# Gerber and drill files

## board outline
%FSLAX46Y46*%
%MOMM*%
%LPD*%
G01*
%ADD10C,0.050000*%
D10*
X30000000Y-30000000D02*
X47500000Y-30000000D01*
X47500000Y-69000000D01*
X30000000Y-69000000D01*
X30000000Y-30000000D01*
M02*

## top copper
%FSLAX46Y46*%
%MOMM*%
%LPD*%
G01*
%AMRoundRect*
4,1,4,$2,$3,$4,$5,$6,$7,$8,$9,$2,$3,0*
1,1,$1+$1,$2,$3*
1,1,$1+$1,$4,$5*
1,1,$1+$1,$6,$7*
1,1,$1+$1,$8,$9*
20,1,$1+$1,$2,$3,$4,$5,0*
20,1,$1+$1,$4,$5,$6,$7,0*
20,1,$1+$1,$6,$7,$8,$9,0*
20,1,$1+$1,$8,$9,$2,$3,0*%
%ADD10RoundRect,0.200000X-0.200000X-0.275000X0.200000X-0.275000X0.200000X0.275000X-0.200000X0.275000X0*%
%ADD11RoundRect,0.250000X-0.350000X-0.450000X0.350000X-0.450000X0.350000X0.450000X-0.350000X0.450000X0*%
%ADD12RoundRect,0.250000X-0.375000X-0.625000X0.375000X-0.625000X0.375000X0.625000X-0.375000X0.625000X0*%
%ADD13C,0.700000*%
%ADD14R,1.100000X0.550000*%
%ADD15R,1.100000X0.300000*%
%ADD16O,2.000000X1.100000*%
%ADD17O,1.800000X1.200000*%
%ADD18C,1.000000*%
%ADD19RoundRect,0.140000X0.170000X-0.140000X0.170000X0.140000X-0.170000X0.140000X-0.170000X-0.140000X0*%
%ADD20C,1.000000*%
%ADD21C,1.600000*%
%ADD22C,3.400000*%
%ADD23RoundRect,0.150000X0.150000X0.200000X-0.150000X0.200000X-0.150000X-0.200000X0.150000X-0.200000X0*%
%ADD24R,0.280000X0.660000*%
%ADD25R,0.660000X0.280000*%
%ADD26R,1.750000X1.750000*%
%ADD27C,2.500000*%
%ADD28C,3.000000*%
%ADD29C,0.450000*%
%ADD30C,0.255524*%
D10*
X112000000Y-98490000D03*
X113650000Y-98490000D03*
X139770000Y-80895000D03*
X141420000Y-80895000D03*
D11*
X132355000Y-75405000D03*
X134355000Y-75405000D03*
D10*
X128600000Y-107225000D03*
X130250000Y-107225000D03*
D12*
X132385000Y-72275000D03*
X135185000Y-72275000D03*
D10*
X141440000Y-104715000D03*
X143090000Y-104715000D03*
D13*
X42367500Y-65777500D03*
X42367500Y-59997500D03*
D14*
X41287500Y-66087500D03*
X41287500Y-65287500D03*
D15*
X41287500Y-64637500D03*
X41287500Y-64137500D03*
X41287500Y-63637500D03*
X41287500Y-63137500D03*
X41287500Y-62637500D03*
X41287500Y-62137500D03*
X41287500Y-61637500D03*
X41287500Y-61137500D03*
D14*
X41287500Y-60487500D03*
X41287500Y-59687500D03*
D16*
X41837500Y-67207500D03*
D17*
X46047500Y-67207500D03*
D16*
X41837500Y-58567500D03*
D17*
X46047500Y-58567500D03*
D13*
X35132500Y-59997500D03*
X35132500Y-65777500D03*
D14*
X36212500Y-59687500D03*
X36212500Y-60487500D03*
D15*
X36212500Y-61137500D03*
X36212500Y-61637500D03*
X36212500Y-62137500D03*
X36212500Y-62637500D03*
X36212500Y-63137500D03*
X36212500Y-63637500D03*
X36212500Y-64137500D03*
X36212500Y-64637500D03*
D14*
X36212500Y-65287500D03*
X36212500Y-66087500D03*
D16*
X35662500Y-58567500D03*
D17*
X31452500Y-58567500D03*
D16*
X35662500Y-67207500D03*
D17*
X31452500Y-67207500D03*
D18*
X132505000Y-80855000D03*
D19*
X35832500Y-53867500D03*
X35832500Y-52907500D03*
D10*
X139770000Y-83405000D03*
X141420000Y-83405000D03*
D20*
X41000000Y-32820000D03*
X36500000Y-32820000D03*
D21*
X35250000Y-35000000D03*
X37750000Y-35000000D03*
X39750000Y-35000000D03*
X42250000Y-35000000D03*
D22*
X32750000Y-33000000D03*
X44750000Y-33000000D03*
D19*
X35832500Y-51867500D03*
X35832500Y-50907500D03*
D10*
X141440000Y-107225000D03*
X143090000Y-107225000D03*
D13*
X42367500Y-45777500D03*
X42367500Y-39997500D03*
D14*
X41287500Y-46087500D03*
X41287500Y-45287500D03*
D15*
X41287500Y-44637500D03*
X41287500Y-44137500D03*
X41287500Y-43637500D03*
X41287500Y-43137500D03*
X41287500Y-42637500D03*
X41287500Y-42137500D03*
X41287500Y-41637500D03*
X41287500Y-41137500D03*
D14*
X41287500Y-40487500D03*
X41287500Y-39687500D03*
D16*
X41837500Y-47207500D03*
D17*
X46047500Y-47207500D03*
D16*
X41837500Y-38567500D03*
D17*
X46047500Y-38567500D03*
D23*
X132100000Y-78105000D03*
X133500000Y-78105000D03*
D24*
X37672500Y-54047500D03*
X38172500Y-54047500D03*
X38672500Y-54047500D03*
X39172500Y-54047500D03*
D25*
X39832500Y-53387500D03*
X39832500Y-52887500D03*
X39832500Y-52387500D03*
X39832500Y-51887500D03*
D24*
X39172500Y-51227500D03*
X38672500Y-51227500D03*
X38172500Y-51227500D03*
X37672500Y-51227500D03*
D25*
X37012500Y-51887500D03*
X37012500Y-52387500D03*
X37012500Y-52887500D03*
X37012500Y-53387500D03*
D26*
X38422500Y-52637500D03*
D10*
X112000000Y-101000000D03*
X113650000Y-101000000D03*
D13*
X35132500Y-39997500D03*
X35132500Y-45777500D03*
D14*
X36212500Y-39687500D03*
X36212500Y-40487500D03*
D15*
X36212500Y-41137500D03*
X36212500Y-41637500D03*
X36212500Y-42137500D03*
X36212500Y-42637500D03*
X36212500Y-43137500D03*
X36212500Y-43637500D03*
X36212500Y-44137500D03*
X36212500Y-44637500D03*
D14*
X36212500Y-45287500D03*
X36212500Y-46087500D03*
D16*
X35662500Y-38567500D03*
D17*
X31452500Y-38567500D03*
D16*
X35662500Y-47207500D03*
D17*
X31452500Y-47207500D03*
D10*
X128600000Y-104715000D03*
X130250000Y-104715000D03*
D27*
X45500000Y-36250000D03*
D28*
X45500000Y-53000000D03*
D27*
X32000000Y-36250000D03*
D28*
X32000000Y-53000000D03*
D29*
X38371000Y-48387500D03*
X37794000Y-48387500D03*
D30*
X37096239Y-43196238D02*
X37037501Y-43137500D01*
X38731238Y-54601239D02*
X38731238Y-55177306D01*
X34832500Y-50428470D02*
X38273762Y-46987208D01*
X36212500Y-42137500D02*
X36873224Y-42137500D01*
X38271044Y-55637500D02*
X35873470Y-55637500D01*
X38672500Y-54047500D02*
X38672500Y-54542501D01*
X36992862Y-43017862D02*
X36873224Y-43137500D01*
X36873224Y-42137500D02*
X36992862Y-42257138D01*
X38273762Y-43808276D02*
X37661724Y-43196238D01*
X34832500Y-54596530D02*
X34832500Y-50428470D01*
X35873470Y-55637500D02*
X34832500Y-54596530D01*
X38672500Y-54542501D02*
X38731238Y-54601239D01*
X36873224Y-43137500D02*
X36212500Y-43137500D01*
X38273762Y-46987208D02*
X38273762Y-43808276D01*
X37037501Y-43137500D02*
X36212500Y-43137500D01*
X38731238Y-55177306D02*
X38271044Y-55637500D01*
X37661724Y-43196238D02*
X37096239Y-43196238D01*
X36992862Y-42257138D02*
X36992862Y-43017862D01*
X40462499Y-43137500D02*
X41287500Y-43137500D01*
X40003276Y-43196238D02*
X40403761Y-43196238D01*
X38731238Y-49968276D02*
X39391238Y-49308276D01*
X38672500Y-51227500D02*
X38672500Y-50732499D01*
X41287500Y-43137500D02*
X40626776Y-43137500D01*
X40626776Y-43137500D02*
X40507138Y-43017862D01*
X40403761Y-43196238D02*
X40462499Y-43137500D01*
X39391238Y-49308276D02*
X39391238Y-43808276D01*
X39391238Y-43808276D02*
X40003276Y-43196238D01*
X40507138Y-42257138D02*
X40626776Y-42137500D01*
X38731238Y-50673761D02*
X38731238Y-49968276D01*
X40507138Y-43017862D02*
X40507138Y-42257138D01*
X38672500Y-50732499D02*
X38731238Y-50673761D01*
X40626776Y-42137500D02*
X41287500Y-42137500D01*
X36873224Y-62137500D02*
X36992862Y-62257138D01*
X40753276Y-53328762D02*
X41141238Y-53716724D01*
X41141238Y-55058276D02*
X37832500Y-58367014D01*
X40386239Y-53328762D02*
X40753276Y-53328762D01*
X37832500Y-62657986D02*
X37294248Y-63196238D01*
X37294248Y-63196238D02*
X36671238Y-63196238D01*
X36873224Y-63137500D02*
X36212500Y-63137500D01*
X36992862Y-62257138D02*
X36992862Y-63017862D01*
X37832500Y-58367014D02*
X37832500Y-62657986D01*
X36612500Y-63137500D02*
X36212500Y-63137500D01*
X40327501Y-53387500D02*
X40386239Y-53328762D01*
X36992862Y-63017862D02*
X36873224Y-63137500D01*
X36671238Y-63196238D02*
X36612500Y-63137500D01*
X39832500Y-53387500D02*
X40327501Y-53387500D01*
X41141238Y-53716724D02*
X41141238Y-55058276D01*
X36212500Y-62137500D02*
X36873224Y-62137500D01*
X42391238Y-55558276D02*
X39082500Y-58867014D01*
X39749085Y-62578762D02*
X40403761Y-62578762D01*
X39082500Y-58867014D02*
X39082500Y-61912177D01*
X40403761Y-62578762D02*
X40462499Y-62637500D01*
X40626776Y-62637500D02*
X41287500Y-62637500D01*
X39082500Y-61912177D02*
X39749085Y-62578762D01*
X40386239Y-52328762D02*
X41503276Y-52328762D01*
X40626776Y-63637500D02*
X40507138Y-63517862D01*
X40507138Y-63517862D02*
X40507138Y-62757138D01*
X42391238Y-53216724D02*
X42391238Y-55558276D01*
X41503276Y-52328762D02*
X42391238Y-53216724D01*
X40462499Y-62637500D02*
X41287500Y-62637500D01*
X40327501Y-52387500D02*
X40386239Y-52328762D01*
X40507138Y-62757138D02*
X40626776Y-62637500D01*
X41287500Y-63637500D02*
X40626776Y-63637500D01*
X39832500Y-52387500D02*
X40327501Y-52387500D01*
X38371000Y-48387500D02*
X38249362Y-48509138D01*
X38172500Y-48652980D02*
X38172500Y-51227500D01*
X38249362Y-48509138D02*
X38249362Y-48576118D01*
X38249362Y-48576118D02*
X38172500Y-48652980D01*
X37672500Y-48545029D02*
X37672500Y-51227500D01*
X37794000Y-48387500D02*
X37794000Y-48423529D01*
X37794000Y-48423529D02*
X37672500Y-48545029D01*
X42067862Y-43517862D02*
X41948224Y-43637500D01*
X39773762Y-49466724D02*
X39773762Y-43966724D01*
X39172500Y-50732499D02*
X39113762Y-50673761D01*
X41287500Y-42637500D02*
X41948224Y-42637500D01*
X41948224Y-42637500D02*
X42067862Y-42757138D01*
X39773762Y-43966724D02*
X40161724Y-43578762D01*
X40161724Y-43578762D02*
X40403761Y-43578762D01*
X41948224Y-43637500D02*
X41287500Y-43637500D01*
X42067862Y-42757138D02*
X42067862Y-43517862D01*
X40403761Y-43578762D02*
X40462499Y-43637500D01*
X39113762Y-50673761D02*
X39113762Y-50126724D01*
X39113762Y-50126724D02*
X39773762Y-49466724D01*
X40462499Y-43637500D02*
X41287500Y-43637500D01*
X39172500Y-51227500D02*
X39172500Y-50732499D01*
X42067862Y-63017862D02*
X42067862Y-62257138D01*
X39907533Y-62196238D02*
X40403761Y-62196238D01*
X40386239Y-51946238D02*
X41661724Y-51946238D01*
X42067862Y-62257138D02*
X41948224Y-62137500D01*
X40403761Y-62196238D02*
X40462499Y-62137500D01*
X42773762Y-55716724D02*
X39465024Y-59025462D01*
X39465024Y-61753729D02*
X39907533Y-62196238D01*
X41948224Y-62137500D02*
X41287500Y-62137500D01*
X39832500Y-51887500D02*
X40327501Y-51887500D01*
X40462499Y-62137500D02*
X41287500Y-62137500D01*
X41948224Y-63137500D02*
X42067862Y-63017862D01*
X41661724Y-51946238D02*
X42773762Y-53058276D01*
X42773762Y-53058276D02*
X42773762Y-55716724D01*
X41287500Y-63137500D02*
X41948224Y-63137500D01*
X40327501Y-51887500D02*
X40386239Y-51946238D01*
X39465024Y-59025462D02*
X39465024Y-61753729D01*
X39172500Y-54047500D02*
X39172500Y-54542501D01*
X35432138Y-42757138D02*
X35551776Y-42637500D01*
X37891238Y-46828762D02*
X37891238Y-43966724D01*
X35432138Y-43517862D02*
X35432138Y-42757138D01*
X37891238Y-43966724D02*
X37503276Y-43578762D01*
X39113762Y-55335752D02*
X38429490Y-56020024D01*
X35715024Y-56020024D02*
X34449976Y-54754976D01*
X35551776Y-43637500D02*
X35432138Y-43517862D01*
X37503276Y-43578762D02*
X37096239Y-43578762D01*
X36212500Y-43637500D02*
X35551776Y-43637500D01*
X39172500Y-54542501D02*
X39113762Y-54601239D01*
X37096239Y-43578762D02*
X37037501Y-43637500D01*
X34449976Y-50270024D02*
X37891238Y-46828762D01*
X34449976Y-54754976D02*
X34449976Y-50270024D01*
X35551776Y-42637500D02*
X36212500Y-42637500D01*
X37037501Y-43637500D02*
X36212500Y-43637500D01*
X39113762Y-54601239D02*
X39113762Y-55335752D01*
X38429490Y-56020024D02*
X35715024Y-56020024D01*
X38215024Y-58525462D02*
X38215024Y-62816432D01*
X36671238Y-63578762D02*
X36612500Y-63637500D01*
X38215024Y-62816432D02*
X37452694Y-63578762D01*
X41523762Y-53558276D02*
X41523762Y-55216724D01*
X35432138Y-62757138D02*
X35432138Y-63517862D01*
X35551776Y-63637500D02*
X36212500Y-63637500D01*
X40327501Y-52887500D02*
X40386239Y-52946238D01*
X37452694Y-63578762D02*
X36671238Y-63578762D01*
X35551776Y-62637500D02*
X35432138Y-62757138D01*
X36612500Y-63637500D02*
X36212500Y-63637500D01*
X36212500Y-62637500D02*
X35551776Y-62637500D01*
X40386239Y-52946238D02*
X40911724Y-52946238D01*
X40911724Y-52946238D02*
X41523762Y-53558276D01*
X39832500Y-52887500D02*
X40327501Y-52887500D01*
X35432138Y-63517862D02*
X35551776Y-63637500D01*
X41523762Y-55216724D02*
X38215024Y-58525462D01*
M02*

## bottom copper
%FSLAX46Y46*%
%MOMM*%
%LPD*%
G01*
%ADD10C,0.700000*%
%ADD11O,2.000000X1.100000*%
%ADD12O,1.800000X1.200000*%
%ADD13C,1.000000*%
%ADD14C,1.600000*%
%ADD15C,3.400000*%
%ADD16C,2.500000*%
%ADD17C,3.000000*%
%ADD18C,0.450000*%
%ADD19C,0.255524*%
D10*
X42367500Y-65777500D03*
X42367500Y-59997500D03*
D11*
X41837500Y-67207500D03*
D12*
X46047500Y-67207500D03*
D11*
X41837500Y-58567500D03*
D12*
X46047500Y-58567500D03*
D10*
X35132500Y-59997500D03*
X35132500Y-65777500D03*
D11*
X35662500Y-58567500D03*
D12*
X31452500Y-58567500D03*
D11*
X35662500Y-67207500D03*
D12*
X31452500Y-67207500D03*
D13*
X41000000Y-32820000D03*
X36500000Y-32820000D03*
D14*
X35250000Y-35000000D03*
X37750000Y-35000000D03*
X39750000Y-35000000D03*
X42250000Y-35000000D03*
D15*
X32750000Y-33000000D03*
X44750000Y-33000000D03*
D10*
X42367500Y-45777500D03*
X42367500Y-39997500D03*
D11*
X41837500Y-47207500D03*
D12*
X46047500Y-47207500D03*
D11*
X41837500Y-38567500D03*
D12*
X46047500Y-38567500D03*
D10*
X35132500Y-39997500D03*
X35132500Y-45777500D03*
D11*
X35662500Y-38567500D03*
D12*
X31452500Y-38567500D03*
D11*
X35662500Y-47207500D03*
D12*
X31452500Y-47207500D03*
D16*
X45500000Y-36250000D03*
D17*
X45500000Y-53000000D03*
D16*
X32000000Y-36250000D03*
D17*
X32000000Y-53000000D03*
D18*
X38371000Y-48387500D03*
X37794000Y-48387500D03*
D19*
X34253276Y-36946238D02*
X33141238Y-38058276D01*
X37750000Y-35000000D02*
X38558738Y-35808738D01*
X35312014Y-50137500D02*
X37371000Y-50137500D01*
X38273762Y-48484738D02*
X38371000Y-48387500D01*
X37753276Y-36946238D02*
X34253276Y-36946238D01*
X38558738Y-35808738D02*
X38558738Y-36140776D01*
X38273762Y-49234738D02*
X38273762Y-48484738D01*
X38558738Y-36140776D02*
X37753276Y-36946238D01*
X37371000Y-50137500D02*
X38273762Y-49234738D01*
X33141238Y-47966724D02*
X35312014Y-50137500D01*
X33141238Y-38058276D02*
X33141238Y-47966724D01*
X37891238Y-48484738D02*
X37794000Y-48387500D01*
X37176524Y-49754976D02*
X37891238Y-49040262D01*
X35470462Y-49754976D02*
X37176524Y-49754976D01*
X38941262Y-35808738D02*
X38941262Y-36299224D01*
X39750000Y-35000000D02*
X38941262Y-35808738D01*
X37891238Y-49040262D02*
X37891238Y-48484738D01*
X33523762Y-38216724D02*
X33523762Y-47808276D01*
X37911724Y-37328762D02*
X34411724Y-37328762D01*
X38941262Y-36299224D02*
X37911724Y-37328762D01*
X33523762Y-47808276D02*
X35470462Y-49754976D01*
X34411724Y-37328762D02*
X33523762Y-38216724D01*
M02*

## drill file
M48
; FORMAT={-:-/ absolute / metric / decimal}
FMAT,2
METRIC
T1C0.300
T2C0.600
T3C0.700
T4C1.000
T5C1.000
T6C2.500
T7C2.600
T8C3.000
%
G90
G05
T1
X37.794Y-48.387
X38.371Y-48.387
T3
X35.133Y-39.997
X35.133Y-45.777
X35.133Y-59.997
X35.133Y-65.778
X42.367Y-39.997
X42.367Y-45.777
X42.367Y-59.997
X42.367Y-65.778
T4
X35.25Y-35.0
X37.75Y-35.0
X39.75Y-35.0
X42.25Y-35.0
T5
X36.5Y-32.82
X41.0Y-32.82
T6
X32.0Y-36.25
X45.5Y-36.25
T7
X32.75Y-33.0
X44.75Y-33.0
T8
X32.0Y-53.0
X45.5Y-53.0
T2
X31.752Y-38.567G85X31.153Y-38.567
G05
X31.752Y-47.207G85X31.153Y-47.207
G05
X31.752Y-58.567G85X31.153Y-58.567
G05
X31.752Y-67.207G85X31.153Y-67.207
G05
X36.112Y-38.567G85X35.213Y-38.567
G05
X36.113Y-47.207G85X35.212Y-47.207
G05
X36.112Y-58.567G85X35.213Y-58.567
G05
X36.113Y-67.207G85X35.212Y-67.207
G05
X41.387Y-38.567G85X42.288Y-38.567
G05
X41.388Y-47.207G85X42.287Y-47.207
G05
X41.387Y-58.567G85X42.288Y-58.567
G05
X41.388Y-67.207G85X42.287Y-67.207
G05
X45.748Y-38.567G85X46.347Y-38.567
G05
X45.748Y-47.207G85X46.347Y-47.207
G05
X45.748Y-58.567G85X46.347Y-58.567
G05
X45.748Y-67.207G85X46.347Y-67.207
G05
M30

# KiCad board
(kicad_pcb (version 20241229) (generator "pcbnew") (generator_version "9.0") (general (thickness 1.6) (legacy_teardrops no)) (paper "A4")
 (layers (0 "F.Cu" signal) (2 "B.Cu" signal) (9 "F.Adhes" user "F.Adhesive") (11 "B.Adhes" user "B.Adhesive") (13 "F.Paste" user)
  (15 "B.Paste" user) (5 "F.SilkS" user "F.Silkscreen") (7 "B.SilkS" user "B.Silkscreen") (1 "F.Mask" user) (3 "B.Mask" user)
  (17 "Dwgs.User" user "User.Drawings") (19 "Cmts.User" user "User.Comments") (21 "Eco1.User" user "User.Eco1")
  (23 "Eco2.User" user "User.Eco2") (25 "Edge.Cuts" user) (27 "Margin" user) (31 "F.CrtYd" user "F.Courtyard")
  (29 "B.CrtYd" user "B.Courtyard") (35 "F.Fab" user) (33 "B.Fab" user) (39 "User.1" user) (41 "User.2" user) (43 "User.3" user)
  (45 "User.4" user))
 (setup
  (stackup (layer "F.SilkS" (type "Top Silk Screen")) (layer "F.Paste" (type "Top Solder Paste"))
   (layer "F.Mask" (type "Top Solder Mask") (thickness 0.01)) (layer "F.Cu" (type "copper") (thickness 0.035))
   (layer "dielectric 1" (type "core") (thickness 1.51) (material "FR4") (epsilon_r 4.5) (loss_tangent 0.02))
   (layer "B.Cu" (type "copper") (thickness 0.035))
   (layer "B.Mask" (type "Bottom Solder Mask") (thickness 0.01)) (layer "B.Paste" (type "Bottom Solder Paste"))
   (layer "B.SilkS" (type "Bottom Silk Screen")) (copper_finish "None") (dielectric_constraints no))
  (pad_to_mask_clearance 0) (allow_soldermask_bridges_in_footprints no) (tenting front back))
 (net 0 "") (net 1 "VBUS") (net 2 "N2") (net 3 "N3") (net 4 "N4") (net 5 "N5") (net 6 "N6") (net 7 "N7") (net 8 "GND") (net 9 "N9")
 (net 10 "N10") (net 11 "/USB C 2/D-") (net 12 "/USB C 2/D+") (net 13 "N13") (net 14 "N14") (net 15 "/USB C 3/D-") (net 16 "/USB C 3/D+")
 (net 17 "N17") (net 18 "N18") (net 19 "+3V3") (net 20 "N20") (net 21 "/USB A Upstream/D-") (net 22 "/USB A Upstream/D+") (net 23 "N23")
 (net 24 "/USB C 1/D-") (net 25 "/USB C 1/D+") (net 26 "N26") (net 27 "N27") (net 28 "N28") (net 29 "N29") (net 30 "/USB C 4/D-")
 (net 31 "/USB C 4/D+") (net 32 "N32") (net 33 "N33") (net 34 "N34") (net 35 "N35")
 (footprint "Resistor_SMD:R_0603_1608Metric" (layer "F.Cu") (at 112.825 98.49)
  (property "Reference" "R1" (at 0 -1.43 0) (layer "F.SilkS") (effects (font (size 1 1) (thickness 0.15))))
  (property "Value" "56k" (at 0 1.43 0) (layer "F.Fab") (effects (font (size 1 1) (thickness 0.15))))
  (pad "1" smd roundrect (at -0.825 0) (size 0.8 0.95) (layers "F.Cu" "F.Mask" "F.Paste") (roundrect_rratio 0.25) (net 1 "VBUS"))
  (pad "2" smd roundrect (at 0.825 0) (size 0.8 0.95) (layers "F.Cu" "F.Mask" "F.Paste") (roundrect_rratio 0.25) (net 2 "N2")))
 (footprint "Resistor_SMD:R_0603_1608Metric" (layer "F.Cu") (at 140.595 80.895)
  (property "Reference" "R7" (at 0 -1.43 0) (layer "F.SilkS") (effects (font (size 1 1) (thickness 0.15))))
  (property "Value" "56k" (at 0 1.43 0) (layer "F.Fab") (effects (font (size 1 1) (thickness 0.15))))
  (pad "1" smd roundrect (at -0.825 0) (size 0.8 0.95) (layers "F.Cu" "F.Mask" "F.Paste") (roundrect_rratio 0.25) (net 1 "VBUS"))
  (pad "2" smd roundrect (at 0.825 0) (size 0.8 0.95) (layers "F.Cu" "F.Mask" "F.Paste") (roundrect_rratio 0.25) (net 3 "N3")))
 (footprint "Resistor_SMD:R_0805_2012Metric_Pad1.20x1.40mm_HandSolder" (layer "F.Cu") (at 133.355 75.405)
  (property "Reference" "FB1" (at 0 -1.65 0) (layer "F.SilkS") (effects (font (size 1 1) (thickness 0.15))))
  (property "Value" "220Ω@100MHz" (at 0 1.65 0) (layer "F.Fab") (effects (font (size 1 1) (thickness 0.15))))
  (pad "1" smd roundrect (at -1 0) (size 1.2 1.4) (layers "F.Cu" "F.Mask" "F.Paste") (roundrect_rratio 0.208333) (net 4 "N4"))
  (pad "2" smd roundrect (at 1 0) (size 1.2 1.4) (layers "F.Cu" "F.Mask" "F.Paste") (roundrect_rratio 0.208333) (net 1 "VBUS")))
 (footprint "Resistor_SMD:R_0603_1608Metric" (layer "F.Cu") (at 129.425 107.225)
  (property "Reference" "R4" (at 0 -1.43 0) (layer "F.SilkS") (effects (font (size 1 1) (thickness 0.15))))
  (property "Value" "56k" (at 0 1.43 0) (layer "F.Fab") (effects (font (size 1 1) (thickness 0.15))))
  (pad "1" smd roundrect (at -0.825 0) (size 0.8 0.95) (layers "F.Cu" "F.Mask" "F.Paste") (roundrect_rratio 0.25) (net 1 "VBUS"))
  (pad "2" smd roundrect (at 0.825 0) (size 0.8 0.95) (layers "F.Cu" "F.Mask" "F.Paste") (roundrect_rratio 0.25) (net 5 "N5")))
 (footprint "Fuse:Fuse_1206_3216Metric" (layer "F.Cu") (at 133.785 72.275)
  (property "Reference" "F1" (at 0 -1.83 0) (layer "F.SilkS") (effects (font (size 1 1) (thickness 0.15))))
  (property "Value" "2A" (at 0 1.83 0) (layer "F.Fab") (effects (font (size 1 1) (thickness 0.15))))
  (pad "1" smd roundrect (at -1.4 0) (size 1.25 1.75) (layers "F.Cu" "F.Mask" "F.Paste") (roundrect_rratio 0.2) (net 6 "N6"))
  (pad "2" smd roundrect (at 1.4 0) (size 1.25 1.75) (layers "F.Cu" "F.Mask" "F.Paste") (roundrect_rratio 0.2) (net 4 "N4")))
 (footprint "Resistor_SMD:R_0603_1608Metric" (layer "F.Cu") (at 142.265 104.715)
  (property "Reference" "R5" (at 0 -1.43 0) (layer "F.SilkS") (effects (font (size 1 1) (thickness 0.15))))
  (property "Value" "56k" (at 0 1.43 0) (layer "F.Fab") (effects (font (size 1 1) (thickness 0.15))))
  (pad "1" smd roundrect (at -0.825 0) (size 0.8 0.95) (layers "F.Cu" "F.Mask" "F.Paste") (roundrect_rratio 0.25) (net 1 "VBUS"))
  (pad "2" smd roundrect (at 0.825 0) (size 0.8 0.95) (layers "F.Cu" "F.Mask" "F.Paste") (roundrect_rratio 0.25) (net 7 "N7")))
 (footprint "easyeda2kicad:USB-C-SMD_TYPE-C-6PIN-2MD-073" (layer "F.Cu") (at 43.6675 62.8875 90)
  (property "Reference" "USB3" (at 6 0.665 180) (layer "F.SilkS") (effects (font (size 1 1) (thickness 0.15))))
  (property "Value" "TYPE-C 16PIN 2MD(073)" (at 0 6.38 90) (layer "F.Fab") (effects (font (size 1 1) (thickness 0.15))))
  (pad "" thru_hole circle (at -2.89 -1.3 90) (size 0.7 0.7) (drill 0.7) (layers "*.Cu" "*.Mask") (remove_unused_layers no))
  (pad "" thru_hole circle (at 2.89 -1.3 90) (size 0.7 0.7) (drill 0.7) (layers "*.Cu" "*.Mask") (remove_unused_layers no))
  (pad "1" smd rect (at -3.2 -2.38 90) (size 0.55 1.1) (layers "F.Cu" "F.Mask" "F.Paste") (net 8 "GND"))
  (pad "2" smd rect (at -2.4 -2.38 90) (size 0.55 1.1) (layers "F.Cu" "F.Mask" "F.Paste") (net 1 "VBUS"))
  (pad "3" smd rect (at -1.75 -2.38 90) (size 0.3 1.1) (layers "F.Cu" "F.Mask" "F.Paste") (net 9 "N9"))
  (pad "4" smd rect (at -1.25 -2.38 90) (size 0.3 1.1) (layers "F.Cu" "F.Mask" "F.Paste") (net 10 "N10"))
  (pad "5" smd rect (at -0.75 -2.38 90) (size 0.3 1.1) (layers "F.Cu" "F.Mask" "F.Paste") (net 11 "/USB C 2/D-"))
  (pad "6" smd rect (at -0.25 -2.38 90) (size 0.3 1.1) (layers "F.Cu" "F.Mask" "F.Paste") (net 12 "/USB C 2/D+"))
  (pad "7" smd rect (at 0.25 -2.38 90) (size 0.3 1.1) (layers "F.Cu" "F.Mask" "F.Paste") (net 11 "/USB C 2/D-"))
  (pad "8" smd rect (at 0.75 -2.38 90) (size 0.3 1.1) (layers "F.Cu" "F.Mask" "F.Paste") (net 12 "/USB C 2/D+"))
  (pad "9" smd rect (at 1.25 -2.38 90) (size 0.3 1.1) (layers "F.Cu" "F.Mask" "F.Paste") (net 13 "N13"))
  (pad "10" smd rect (at 1.75 -2.38 90) (size 0.3 1.1) (layers "F.Cu" "F.Mask" "F.Paste") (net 5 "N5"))
  (pad "11" smd rect (at 2.4 -2.38 90) (size 0.55 1.1) (layers "F.Cu" "F.Mask" "F.Paste") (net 1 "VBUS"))
  (pad "12" smd rect (at 3.2 -2.38 90) (size 0.55 1.1) (layers "F.Cu" "F.Mask" "F.Paste") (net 8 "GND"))
  (pad "13" thru_hole oval (at -4.32 -1.83 90) (size 1.1 2) (drill oval 0.599999 1.499997) (layers "*.Cu" "*.Mask")
   (remove_unused_layers no) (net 8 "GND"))
  (pad "13" thru_hole oval (at -4.32 2.38 90) (size 1.2 1.8) (drill oval 0.599999 1.199998) (layers "*.Cu" "*.Mask")
   (remove_unused_layers no) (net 8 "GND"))
  (pad "14" thru_hole oval (at 4.32 -1.83 90) (size 1.1 2) (drill oval 0.599999 1.500022) (layers "*.Cu" "*.Mask") (remove_unused_layers no)
   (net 8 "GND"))
  (pad "14" thru_hole oval (at 4.32 2.38 90) (size 1.2 1.8) (drill oval 0.599999 1.199998) (layers "*.Cu" "*.Mask")
   (remove_unused_layers no) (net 8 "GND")))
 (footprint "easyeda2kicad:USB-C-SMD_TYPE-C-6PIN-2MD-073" (layer "F.Cu") (at 33.8325 62.8875 -90)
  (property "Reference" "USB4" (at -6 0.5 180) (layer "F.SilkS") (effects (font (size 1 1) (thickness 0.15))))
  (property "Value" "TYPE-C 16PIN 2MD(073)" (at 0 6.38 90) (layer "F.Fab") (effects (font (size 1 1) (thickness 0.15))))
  (pad "" thru_hole circle (at -2.89 -1.3 270) (size 0.7 0.7) (drill 0.7) (layers "*.Cu" "*.Mask") (remove_unused_layers no))
  (pad "" thru_hole circle (at 2.89 -1.3 270) (size 0.7 0.7) (drill 0.7) (layers "*.Cu" "*.Mask") (remove_unused_layers no))
  (pad "1" smd rect (at -3.2 -2.38 270) (size 0.55 1.1) (layers "F.Cu" "F.Mask" "F.Paste") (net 8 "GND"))
  (pad "2" smd rect (at -2.4 -2.38 270) (size 0.55 1.1) (layers "F.Cu" "F.Mask" "F.Paste") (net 1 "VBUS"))
  (pad "3" smd rect (at -1.75 -2.38 270) (size 0.3 1.1) (layers "F.Cu" "F.Mask" "F.Paste") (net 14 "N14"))
  (pad "4" smd rect (at -1.25 -2.38 270) (size 0.3 1.1) (layers "F.Cu" "F.Mask" "F.Paste") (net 7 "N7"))
  (pad "5" smd rect (at -0.75 -2.38 270) (size 0.3 1.1) (layers "F.Cu" "F.Mask" "F.Paste") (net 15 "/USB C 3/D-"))
  (pad "6" smd rect (at -0.25 -2.38 270) (size 0.3 1.1) (layers "F.Cu" "F.Mask" "F.Paste") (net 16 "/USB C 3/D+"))
  (pad "7" smd rect (at 0.25 -2.38 270) (size 0.3 1.1) (layers "F.Cu" "F.Mask" "F.Paste") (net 15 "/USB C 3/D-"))
  (pad "8" smd rect (at 0.75 -2.38 270) (size 0.3 1.1) (layers "F.Cu" "F.Mask" "F.Paste") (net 16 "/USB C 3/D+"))
  (pad "9" smd rect (at 1.25 -2.38 270) (size 0.3 1.1) (layers "F.Cu" "F.Mask" "F.Paste") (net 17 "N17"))
  (pad "10" smd rect (at 1.75 -2.38 270) (size 0.3 1.1) (layers "F.Cu" "F.Mask" "F.Paste") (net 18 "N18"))
  (pad "11" smd rect (at 2.4 -2.38 270) (size 0.55 1.1) (layers "F.Cu" "F.Mask" "F.Paste") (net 1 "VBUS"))
  (pad "12" smd rect (at 3.2 -2.38 270) (size 0.55 1.1) (layers "F.Cu" "F.Mask" "F.Paste") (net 8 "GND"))
  (pad "13" thru_hole oval (at -4.32 -1.83 270) (size 1.1 2) (drill oval 0.599999 1.499997) (layers "*.Cu" "*.Mask")
   (remove_unused_layers no) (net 8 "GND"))
  (pad "13" thru_hole oval (at -4.32 2.38 270) (size 1.2 1.8) (drill oval 0.599999 1.199998) (layers "*.Cu" "*.Mask")
   (remove_unused_layers no) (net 8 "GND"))
  (pad "14" thru_hole oval (at 4.32 -1.83 270) (size 1.1 2) (drill oval 0.599999 1.500022) (layers "*.Cu" "*.Mask")
   (remove_unused_layers no) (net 8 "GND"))
  (pad "14" thru_hole oval (at 4.32 2.38 270) (size 1.2 1.8) (drill oval 0.599999 1.199998) (layers "*.Cu" "*.Mask")
   (remove_unused_layers no) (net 8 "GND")))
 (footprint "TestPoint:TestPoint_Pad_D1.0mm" (layer "F.Cu") (at 132.505 80.855)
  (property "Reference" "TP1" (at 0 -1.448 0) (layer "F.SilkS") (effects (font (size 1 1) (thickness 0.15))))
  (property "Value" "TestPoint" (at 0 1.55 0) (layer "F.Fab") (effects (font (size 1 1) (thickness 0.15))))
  (pad "1" smd circle (at 0 0) (size 1 1) (layers "F.Cu" "F.Mask") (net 1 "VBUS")))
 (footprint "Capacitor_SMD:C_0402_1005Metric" (layer "F.Cu") (at 35.8325 53.3875 90)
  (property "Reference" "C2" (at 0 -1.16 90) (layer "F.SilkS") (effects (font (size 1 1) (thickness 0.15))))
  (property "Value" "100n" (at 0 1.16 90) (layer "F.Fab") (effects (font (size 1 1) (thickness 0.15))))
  (pad "1" smd roundrect (at -0.48 0 90) (size 0.56 0.62) (layers "F.Cu" "F.Mask" "F.Paste") (roundrect_rratio 0.25) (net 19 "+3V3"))
  (pad "2" smd roundrect (at 0.48 0 90) (size 0.56 0.62) (layers "F.Cu" "F.Mask" "F.Paste") (roundrect_rratio 0.25) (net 8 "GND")))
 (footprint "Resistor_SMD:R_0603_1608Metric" (layer "F.Cu") (at 140.595 83.405)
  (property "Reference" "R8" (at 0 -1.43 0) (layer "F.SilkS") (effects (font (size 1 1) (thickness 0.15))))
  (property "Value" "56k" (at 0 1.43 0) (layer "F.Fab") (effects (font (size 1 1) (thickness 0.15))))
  (pad "1" smd roundrect (at -0.825 0) (size 0.8 0.95) (layers "F.Cu" "F.Mask" "F.Paste") (roundrect_rratio 0.25) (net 1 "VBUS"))
  (pad "2" smd roundrect (at 0.825 0) (size 0.8 0.95) (layers "F.Cu" "F.Mask" "F.Paste") (roundrect_rratio 0.25) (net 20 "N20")))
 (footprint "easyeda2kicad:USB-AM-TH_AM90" (layer "F.Cu") (at 38.75 34 180)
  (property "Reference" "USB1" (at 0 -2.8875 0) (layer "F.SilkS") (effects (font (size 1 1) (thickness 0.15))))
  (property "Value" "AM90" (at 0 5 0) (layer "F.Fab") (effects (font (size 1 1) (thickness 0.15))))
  (pad "" thru_hole circle (at -2.25 1.18 180) (size 1 1) (drill 1) (layers "*.Cu" "*.Mask") (remove_unused_layers no))
  (pad "" thru_hole circle (at 2.25 1.18 180) (size 1 1) (drill 1) (layers "*.Cu" "*.Mask") (remove_unused_layers no))
  (pad "1" thru_hole circle (at 3.5 -1 90) (size 1.6 1.6) (drill 0.999998) (layers "*.Cu" "*.Mask") (remove_unused_layers no) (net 6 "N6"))
  (pad "2" thru_hole circle (at 1 -1 90) (size 1.6 1.6) (drill 0.999998) (layers "*.Cu" "*.Mask") (remove_unused_layers no)
   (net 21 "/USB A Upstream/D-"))
  (pad "3" thru_hole circle (at -1 -1 90) (size 1.6 1.6) (drill 0.999998) (layers "*.Cu" "*.Mask") (remove_unused_layers no)
   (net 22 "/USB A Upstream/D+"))
  (pad "4" thru_hole circle (at -3.5 -1 90) (size 1.6 1.6) (drill 0.999998) (layers "*.Cu" "*.Mask") (remove_unused_layers no) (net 8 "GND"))
  (pad "MH1" thru_hole circle (at 6 1 90) (size 3.4 3.4) (drill 2.599995) (layers "*.Cu" "*.Mask") (remove_unused_layers no) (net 8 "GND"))
  (pad "MH2" thru_hole circle (at -6 1 90) (size 3.4 3.4) (drill 2.599995) (layers "*.Cu" "*.Mask") (remove_unused_layers no) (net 8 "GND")))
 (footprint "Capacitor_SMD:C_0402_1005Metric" (layer "F.Cu") (at 35.8325 51.3875 90)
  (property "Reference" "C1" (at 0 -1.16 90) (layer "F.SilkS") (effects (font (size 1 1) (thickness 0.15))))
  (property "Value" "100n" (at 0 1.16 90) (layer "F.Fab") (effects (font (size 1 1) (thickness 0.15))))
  (pad "1" smd roundrect (at -0.48 0 90) (size 0.56 0.62) (layers "F.Cu" "F.Mask" "F.Paste") (roundrect_rratio 0.25) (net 1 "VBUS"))
  (pad "2" smd roundrect (at 0.48 0 90) (size 0.56 0.62) (layers "F.Cu" "F.Mask" "F.Paste") (roundrect_rratio 0.25) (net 8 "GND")))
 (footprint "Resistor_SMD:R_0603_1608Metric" (layer "F.Cu") (at 142.265 107.225)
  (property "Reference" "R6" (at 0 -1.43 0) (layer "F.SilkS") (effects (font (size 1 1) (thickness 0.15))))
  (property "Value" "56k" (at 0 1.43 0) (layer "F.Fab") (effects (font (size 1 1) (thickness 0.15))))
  (pad "1" smd roundrect (at -0.825 0) (size 0.8 0.95) (layers "F.Cu" "F.Mask" "F.Paste") (roundrect_rratio 0.25) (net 1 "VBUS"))
  (pad "2" smd roundrect (at 0.825 0) (size 0.8 0.95) (layers "F.Cu" "F.Mask" "F.Paste") (roundrect_rratio 0.25) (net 18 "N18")))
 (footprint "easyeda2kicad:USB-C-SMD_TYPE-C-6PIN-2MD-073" (layer "F.Cu") (at 43.6675 42.8875 90)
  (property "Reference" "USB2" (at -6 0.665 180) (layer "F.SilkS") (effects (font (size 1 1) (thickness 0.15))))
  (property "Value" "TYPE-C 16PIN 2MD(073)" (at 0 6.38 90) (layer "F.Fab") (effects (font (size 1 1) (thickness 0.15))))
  (pad "" thru_hole circle (at -2.89 -1.3 90) (size 0.7 0.7) (drill 0.7) (layers "*.Cu" "*.Mask") (remove_unused_layers no))
  (pad "" thru_hole circle (at 2.89 -1.3 90) (size 0.7 0.7) (drill 0.7) (layers "*.Cu" "*.Mask") (remove_unused_layers no))
  (pad "1" smd rect (at -3.2 -2.38 90) (size 0.55 1.1) (layers "F.Cu" "F.Mask" "F.Paste") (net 8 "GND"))
  (pad "2" smd rect (at -2.4 -2.38 90) (size 0.55 1.1) (layers "F.Cu" "F.Mask" "F.Paste") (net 1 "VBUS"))
  (pad "3" smd rect (at -1.75 -2.38 90) (size 0.3 1.1) (layers "F.Cu" "F.Mask" "F.Paste") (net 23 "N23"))
  (pad "4" smd rect (at -1.25 -2.38 90) (size 0.3 1.1) (layers "F.Cu" "F.Mask" "F.Paste") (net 2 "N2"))
  (pad "5" smd rect (at -0.75 -2.38 90) (size 0.3 1.1) (layers "F.Cu" "F.Mask" "F.Paste") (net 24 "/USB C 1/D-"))
  (pad "6" smd rect (at -0.25 -2.38 90) (size 0.3 1.1) (layers "F.Cu" "F.Mask" "F.Paste") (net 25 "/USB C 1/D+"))
  (pad "7" smd rect (at 0.25 -2.38 90) (size 0.3 1.1) (layers "F.Cu" "F.Mask" "F.Paste") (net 24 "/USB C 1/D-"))
  (pad "8" smd rect (at 0.75 -2.38 90) (size 0.3 1.1) (layers "F.Cu" "F.Mask" "F.Paste") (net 25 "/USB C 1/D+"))
  (pad "9" smd rect (at 1.25 -2.38 90) (size 0.3 1.1) (layers "F.Cu" "F.Mask" "F.Paste") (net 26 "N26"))
  (pad "10" smd rect (at 1.75 -2.38 90) (size 0.3 1.1) (layers "F.Cu" "F.Mask" "F.Paste") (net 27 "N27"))
  (pad "11" smd rect (at 2.4 -2.38 90) (size 0.55 1.1) (layers "F.Cu" "F.Mask" "F.Paste") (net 1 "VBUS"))
  (pad "12" smd rect (at 3.2 -2.38 90) (size 0.55 1.1) (layers "F.Cu" "F.Mask" "F.Paste") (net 8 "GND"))
  (pad "13" thru_hole oval (at -4.32 -1.83 90) (size 1.1 2) (drill oval 0.599999 1.499997) (layers "*.Cu" "*.Mask")
   (remove_unused_layers no) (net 8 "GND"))
  (pad "13" thru_hole oval (at -4.32 2.38 90) (size 1.2 1.8) (drill oval 0.599999 1.199998) (layers "*.Cu" "*.Mask")
   (remove_unused_layers no) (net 8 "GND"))
  (pad "14" thru_hole oval (at 4.32 -1.83 90) (size 1.1 2) (drill oval 0.599999 1.500022) (layers "*.Cu" "*.Mask") (remove_unused_layers no)
   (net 8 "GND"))
  (pad "14" thru_hole oval (at 4.32 2.38 90) (size 1.2 1.8) (drill oval 0.599999 1.199998) (layers "*.Cu" "*.Mask")
   (remove_unused_layers no) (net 8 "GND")))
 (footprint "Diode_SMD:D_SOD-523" (layer "F.Cu") (at 132.8 78.105)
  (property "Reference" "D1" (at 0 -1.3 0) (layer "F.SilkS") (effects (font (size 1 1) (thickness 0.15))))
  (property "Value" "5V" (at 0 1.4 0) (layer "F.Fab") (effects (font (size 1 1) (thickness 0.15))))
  (pad "1" smd roundrect (at -0.7 0 180) (size 0.6 0.7) (layers "F.Cu" "F.Mask" "F.Paste") (roundrect_rratio 0.25) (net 4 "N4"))
  (pad "2" smd roundrect (at 0.7 0 180) (size 0.6 0.7) (layers "F.Cu" "F.Mask" "F.Paste") (roundrect_rratio 0.25) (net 8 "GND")))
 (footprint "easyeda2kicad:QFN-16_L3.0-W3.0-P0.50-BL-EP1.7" (layer "F.Cu") (at 38.4225 52.6375)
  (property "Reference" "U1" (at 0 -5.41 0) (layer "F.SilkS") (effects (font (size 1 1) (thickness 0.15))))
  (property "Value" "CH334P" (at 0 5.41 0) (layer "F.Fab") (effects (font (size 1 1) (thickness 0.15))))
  (pad "1" smd rect (at -0.75 1.41) (size 0.28 0.66) (layers "F.Cu" "F.Mask" "F.Paste") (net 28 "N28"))
  (pad "2" smd rect (at -0.25 1.41) (size 0.28 0.66) (layers "F.Cu" "F.Mask" "F.Paste") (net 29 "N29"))
  (pad "3" smd rect (at 0.25 1.41) (size 0.28 0.66) (layers "F.Cu" "F.Mask" "F.Paste") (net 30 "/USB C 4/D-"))
  (pad "4" smd rect (at 0.75 1.41) (size 0.28 0.66) (layers "F.Cu" "F.Mask" "F.Paste") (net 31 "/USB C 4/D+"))
  (pad "5" smd rect (at 1.41 0.75) (size 0.66 0.28) (layers "F.Cu" "F.Mask" "F.Paste") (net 15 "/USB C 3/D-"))
  (pad "6" smd rect (at 1.41 0.25) (size 0.66 0.28) (layers "F.Cu" "F.Mask" "F.Paste") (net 16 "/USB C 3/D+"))
  (pad "7" smd rect (at 1.41 -0.25) (size 0.66 0.28) (layers "F.Cu" "F.Mask" "F.Paste") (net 11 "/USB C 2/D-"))
  (pad "8" smd rect (at 1.41 -0.75) (size 0.66 0.28) (layers "F.Cu" "F.Mask" "F.Paste") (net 12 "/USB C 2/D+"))
  (pad "9" smd rect (at 0.75 -1.41) (size 0.28 0.66) (layers "F.Cu" "F.Mask" "F.Paste") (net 24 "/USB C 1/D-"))
  (pad "10" smd rect (at 0.25 -1.41) (size 0.28 0.66) (layers "F.Cu" "F.Mask" "F.Paste") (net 25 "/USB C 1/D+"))
  (pad "11" smd rect (at -0.25 -1.41) (size 0.28 0.66) (layers "F.Cu" "F.Mask" "F.Paste") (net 21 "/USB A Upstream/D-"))
  (pad "12" smd rect (at -0.75 -1.41) (size 0.28 0.66) (layers "F.Cu" "F.Mask" "F.Paste") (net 22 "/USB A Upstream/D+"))
  (pad "13" smd rect (at -1.41 -0.75) (size 0.66 0.28) (layers "F.Cu" "F.Mask" "F.Paste") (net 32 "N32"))
  (pad "14" smd rect (at -1.41 -0.25) (size 0.66 0.28) (layers "F.Cu" "F.Mask" "F.Paste") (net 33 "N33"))
  (pad "15" smd rect (at -1.41 0.25) (size 0.66 0.28) (layers "F.Cu" "F.Mask" "F.Paste") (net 1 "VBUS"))
  (pad "16" smd rect (at -1.41 0.75) (size 0.66 0.28) (layers "F.Cu" "F.Mask" "F.Paste") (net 19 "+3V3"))
  (pad "17" smd rect (at 0 0) (size 1.75 1.75) (layers "F.Cu" "F.Mask" "F.Paste") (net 8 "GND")))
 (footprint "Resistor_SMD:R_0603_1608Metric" (layer "F.Cu") (at 112.825 101)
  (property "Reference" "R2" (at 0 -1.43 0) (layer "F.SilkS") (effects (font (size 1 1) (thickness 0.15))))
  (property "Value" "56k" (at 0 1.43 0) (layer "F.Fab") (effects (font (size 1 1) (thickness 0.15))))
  (pad "1" smd roundrect (at -0.825 0) (size 0.8 0.95) (layers "F.Cu" "F.Mask" "F.Paste") (roundrect_rratio 0.25) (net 1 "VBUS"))
  (pad "2" smd roundrect (at 0.825 0) (size 0.8 0.95) (layers "F.Cu" "F.Mask" "F.Paste") (roundrect_rratio 0.25) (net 27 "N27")))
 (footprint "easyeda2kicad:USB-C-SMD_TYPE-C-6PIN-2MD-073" (layer "F.Cu") (at 33.8325 42.8875 -90)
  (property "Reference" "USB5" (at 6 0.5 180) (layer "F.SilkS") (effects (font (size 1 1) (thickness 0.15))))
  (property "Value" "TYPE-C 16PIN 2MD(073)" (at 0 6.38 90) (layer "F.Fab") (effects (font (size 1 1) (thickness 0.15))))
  (pad "" thru_hole circle (at -2.89 -1.3 270) (size 0.7 0.7) (drill 0.7) (layers "*.Cu" "*.Mask") (remove_unused_layers no))
  (pad "" thru_hole circle (at 2.89 -1.3 270) (size 0.7 0.7) (drill 0.7) (layers "*.Cu" "*.Mask") (remove_unused_layers no))
  (pad "1" smd rect (at -3.2 -2.38 270) (size 0.55 1.1) (layers "F.Cu" "F.Mask" "F.Paste") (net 8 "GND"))
  (pad "2" smd rect (at -2.4 -2.38 270) (size 0.55 1.1) (layers "F.Cu" "F.Mask" "F.Paste") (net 1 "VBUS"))
  (pad "3" smd rect (at -1.75 -2.38 270) (size 0.3 1.1) (layers "F.Cu" "F.Mask" "F.Paste") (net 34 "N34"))
  (pad "4" smd rect (at -1.25 -2.38 270) (size 0.3 1.1) (layers "F.Cu" "F.Mask" "F.Paste") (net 3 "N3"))
  (pad "5" smd rect (at -0.75 -2.38 270) (size 0.3 1.1) (layers "F.Cu" "F.Mask" "F.Paste") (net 30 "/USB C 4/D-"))
  (pad "6" smd rect (at -0.25 -2.38 270) (size 0.3 1.1) (layers "F.Cu" "F.Mask" "F.Paste") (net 31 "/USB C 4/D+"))
  (pad "7" smd rect (at 0.25 -2.38 270) (size 0.3 1.1) (layers "F.Cu" "F.Mask" "F.Paste") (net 30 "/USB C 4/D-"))
  (pad "8" smd rect (at 0.75 -2.38 270) (size 0.3 1.1) (layers "F.Cu" "F.Mask" "F.Paste") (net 31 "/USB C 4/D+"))
  (pad "9" smd rect (at 1.25 -2.38 270) (size 0.3 1.1) (layers "F.Cu" "F.Mask" "F.Paste") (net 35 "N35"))
  (pad "10" smd rect (at 1.75 -2.38 270) (size 0.3 1.1) (layers "F.Cu" "F.Mask" "F.Paste") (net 20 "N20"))
  (pad "11" smd rect (at 2.4 -2.38 270) (size 0.55 1.1) (layers "F.Cu" "F.Mask" "F.Paste") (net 1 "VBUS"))
  (pad "12" smd rect (at 3.2 -2.38 270) (size 0.55 1.1) (layers "F.Cu" "F.Mask" "F.Paste") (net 8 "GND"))
  (pad "13" thru_hole oval (at -4.32 -1.83 270) (size 1.1 2) (drill oval 0.599999 1.499997) (layers "*.Cu" "*.Mask")
   (remove_unused_layers no) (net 8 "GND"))
  (pad "13" thru_hole oval (at -4.32 2.38 270) (size 1.2 1.8) (drill oval 0.599999 1.199998) (layers "*.Cu" "*.Mask")
   (remove_unused_layers no) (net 8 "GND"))
  (pad "14" thru_hole oval (at 4.32 -1.83 270) (size 1.1 2) (drill oval 0.599999 1.500022) (layers "*.Cu" "*.Mask")
   (remove_unused_layers no) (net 8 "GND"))
  (pad "14" thru_hole oval (at 4.32 2.38 270) (size 1.2 1.8) (drill oval 0.599999 1.199998) (layers "*.Cu" "*.Mask")
   (remove_unused_layers no) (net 8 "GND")))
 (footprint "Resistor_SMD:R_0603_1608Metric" (layer "F.Cu") (at 129.425 104.715)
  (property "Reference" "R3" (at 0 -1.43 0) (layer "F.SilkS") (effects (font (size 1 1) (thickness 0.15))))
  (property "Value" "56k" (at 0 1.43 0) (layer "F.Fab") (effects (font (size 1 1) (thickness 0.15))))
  (pad "1" smd roundrect (at -0.825 0) (size 0.8 0.95) (layers "F.Cu" "F.Mask" "F.Paste") (roundrect_rratio 0.25) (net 1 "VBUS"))
  (pad "2" smd roundrect (at 0.825 0) (size 0.8 0.95) (layers "F.Cu" "F.Mask" "F.Paste") (roundrect_rratio 0.25) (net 10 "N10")))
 (gr_rect (start 30 30) (end 47.5 69) (stroke (width 0.05) (type default)) (fill no) (layer "Edge.Cuts"))
 (via (at 45.5 36.25) (size 2.5) (drill 2.5) (layers "F.Cu" "B.Cu") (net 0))
 (via (at 45.5 53) (size 3) (drill 3) (layers "F.Cu" "B.Cu") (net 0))
 (via (at 32 36.25) (size 2.5) (drill 2.5) (layers "F.Cu" "B.Cu") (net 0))
 (via (at 32 53) (size 3) (drill 3) (layers "F.Cu" "B.Cu") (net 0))
 (segment (start 37.096239 43.196238) (end 37.037501 43.1375) (width 0.255524) (layer "F.Cu") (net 30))
 (segment (start 38.731238 54.601239) (end 38.731238 55.177306) (width 0.255524) (layer "F.Cu") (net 30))
 (segment (start 34.8325 50.42847) (end 38.273762 46.987208) (width 0.255524) (layer "F.Cu") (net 30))
 (segment (start 36.2125 42.1375) (end 36.873224 42.1375) (width 0.255524) (layer "F.Cu") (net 30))
 (segment (start 38.271044 55.6375) (end 35.87347 55.6375) (width 0.255524) (layer "F.Cu") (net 30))
 (segment (start 38.6725 54.0475) (end 38.6725 54.542501) (width 0.255524) (layer "F.Cu") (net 30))
 (segment (start 36.992862 43.017862) (end 36.873224 43.1375) (width 0.255524) (layer "F.Cu") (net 30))
 (segment (start 36.873224 42.1375) (end 36.992862 42.257138) (width 0.255524) (layer "F.Cu") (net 30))
 (segment (start 38.273762 43.808276) (end 37.661724 43.196238) (width 0.255524) (layer "F.Cu") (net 30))
 (segment (start 34.8325 54.59653) (end 34.8325 50.42847) (width 0.255524) (layer "F.Cu") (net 30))
 (segment (start 35.87347 55.6375) (end 34.8325 54.59653) (width 0.255524) (layer "F.Cu") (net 30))
 (segment (start 38.6725 54.542501) (end 38.731238 54.601239) (width 0.255524) (layer "F.Cu") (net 30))
 (segment (start 36.873224 43.1375) (end 36.2125 43.1375) (width 0.255524) (layer "F.Cu") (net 30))
 (segment (start 38.273762 46.987208) (end 38.273762 43.808276) (width 0.255524) (layer "F.Cu") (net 30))
 (segment (start 37.037501 43.1375) (end 36.2125 43.1375) (width 0.255524) (layer "F.Cu") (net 30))
 (segment (start 38.731238 55.177306) (end 38.271044 55.6375) (width 0.255524) (layer "F.Cu") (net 30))
 (segment (start 37.661724 43.196238) (end 37.096239 43.196238) (width 0.255524) (layer "F.Cu") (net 30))
 (segment (start 36.992862 42.257138) (end 36.992862 43.017862) (width 0.255524) (layer "F.Cu") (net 30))
 (segment (start 40.462499 43.1375) (end 41.2875 43.1375) (width 0.255524) (layer "F.Cu") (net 25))
 (segment (start 40.003276 43.196238) (end 40.403761 43.196238) (width 0.255524) (layer "F.Cu") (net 25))
 (segment (start 38.731238 49.968276) (end 39.391238 49.308276) (width 0.255524) (layer "F.Cu") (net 25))
 (segment (start 38.6725 51.2275) (end 38.6725 50.732499) (width 0.255524) (layer "F.Cu") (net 25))
 (segment (start 41.2875 43.1375) (end 40.626776 43.1375) (width 0.255524) (layer "F.Cu") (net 25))
 (segment (start 40.626776 43.1375) (end 40.507138 43.017862) (width 0.255524) (layer "F.Cu") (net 25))
 (segment (start 40.403761 43.196238) (end 40.462499 43.1375) (width 0.255524) (layer "F.Cu") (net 25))
 (segment (start 39.391238 49.308276) (end 39.391238 43.808276) (width 0.255524) (layer "F.Cu") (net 25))
 (segment (start 39.391238 43.808276) (end 40.003276 43.196238) (width 0.255524) (layer "F.Cu") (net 25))
 (segment (start 40.507138 42.257138) (end 40.626776 42.1375) (width 0.255524) (layer "F.Cu") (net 25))
 (segment (start 38.731238 50.673761) (end 38.731238 49.968276) (width 0.255524) (layer "F.Cu") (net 25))
 (segment (start 40.507138 43.017862) (end 40.507138 42.257138) (width 0.255524) (layer "F.Cu") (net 25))
 (segment (start 38.6725 50.732499) (end 38.731238 50.673761) (width 0.255524) (layer "F.Cu") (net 25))
 (segment (start 40.626776 42.1375) (end 41.2875 42.1375) (width 0.255524) (layer "F.Cu") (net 25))
 (segment (start 36.873224 62.1375) (end 36.992862 62.257138) (width 0.255524) (layer "F.Cu") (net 15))
 (segment (start 40.753276 53.328762) (end 41.141238 53.716724) (width 0.255524) (layer "F.Cu") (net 15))
 (segment (start 41.141238 55.058276) (end 37.8325 58.367014) (width 0.255524) (layer "F.Cu") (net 15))
 (segment (start 40.386239 53.328762) (end 40.753276 53.328762) (width 0.255524) (layer "F.Cu") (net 15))
 (segment (start 37.8325 62.657986) (end 37.294248 63.196238) (width 0.255524) (layer "F.Cu") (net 15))
 (segment (start 37.294248 63.196238) (end 36.671238 63.196238) (width 0.255524) (layer "F.Cu") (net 15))
 (segment (start 36.873224 63.1375) (end 36.2125 63.1375) (width 0.255524) (layer "F.Cu") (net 15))
 (segment (start 36.992862 62.257138) (end 36.992862 63.017862) (width 0.255524) (layer "F.Cu") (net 15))
 (segment (start 37.8325 58.367014) (end 37.8325 62.657986) (width 0.255524) (layer "F.Cu") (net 15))
 (segment (start 36.6125 63.1375) (end 36.2125 63.1375) (width 0.255524) (layer "F.Cu") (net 15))
 (segment (start 40.327501 53.3875) (end 40.386239 53.328762) (width 0.255524) (layer "F.Cu") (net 15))
 (segment (start 36.992862 63.017862) (end 36.873224 63.1375) (width 0.255524) (layer "F.Cu") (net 15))
 (segment (start 36.671238 63.196238) (end 36.6125 63.1375) (width 0.255524) (layer "F.Cu") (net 15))
 (segment (start 39.8325 53.3875) (end 40.327501 53.3875) (width 0.255524) (layer "F.Cu") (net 15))
 (segment (start 41.141238 53.716724) (end 41.141238 55.058276) (width 0.255524) (layer "F.Cu") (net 15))
 (segment (start 36.2125 62.1375) (end 36.873224 62.1375) (width 0.255524) (layer "F.Cu") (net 15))
 (segment (start 42.391238 55.558276) (end 39.0825 58.867014) (width 0.255524) (layer "F.Cu") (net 11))
 (segment (start 39.749085 62.578762) (end 40.403761 62.578762) (width 0.255524) (layer "F.Cu") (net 11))
 (segment (start 39.0825 58.867014) (end 39.0825 61.912177) (width 0.255524) (layer "F.Cu") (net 11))
 (segment (start 40.403761 62.578762) (end 40.462499 62.6375) (width 0.255524) (layer "F.Cu") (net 11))
 (segment (start 40.626776 62.6375) (end 41.2875 62.6375) (width 0.255524) (layer "F.Cu") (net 11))
 (segment (start 39.0825 61.912177) (end 39.749085 62.578762) (width 0.255524) (layer "F.Cu") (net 11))
 (segment (start 40.386239 52.328762) (end 41.503276 52.328762) (width 0.255524) (layer "F.Cu") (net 11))
 (segment (start 40.626776 63.6375) (end 40.507138 63.517862) (width 0.255524) (layer "F.Cu") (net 11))
 (segment (start 40.507138 63.517862) (end 40.507138 62.757138) (width 0.255524) (layer "F.Cu") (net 11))
 (segment (start 42.391238 53.216724) (end 42.391238 55.558276) (width 0.255524) (layer "F.Cu") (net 11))
 (segment (start 41.503276 52.328762) (end 42.391238 53.216724) (width 0.255524) (layer "F.Cu") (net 11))
 (segment (start 40.462499 62.6375) (end 41.2875 62.6375) (width 0.255524) (layer "F.Cu") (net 11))
 (segment (start 40.327501 52.3875) (end 40.386239 52.328762) (width 0.255524) (layer "F.Cu") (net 11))
 (segment (start 40.507138 62.757138) (end 40.626776 62.6375) (width 0.255524) (layer "F.Cu") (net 11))
 (segment (start 41.2875 63.6375) (end 40.626776 63.6375) (width 0.255524) (layer "F.Cu") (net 11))
 (segment (start 39.8325 52.3875) (end 40.327501 52.3875) (width 0.255524) (layer "F.Cu") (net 11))
 (segment (start 38.371 48.3875) (end 38.249362 48.509138) (width 0.255524) (layer "F.Cu") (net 21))
 (segment (start 38.1725 48.65298) (end 38.1725 51.2275) (width 0.255524) (layer "F.Cu") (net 21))
 (segment (start 38.249362 48.509138) (end 38.249362 48.576118) (width 0.255524) (layer "F.Cu") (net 21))
 (segment (start 38.249362 48.576118) (end 38.1725 48.65298) (width 0.255524) (layer "F.Cu") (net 21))
 (via (at 38.371 48.3875) (size 0.45) (drill 0.3) (layers "F.Cu" "B.Cu") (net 21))
 (segment (start 34.253276 36.946238) (end 33.141238 38.058276) (width 0.255524) (layer "B.Cu") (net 21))
 (segment (start 37.75 35) (end 38.558738 35.808738) (width 0.255524) (layer "B.Cu") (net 21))
 (segment (start 35.312014 50.1375) (end 37.371 50.1375) (width 0.255524) (layer "B.Cu") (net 21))
 (segment (start 38.273762 48.484738) (end 38.371 48.3875) (width 0.255524) (layer "B.Cu") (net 21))
 (segment (start 37.753276 36.946238) (end 34.253276 36.946238) (width 0.255524) (layer "B.Cu") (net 21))
 (segment (start 38.558738 35.808738) (end 38.558738 36.140776) (width 0.255524) (layer "B.Cu") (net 21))
 (segment (start 38.273762 49.234738) (end 38.273762 48.484738) (width 0.255524) (layer "B.Cu") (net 21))
 (segment (start 38.558738 36.140776) (end 37.753276 36.946238) (width 0.255524) (layer "B.Cu") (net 21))
 (segment (start 37.371 50.1375) (end 38.273762 49.234738) (width 0.255524) (layer "B.Cu") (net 21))
 (segment (start 33.141238 47.966724) (end 35.312014 50.1375) (width 0.255524) (layer "B.Cu") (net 21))
 (segment (start 33.141238 38.058276) (end 33.141238 47.966724) (width 0.255524) (layer "B.Cu") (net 21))
 (segment (start 37.6725 48.545029) (end 37.6725 51.2275) (width 0.255524) (layer "F.Cu") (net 22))
 (segment (start 37.794 48.3875) (end 37.794 48.423529) (width 0.255524) (layer "F.Cu") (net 22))
 (segment (start 37.794 48.423529) (end 37.6725 48.545029) (width 0.255524) (layer "F.Cu") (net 22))
 (via (at 37.794 48.3875) (size 0.45) (drill 0.3) (layers "F.Cu" "B.Cu") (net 22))
 (segment (start 37.891238 48.484738) (end 37.794 48.3875) (width 0.255524) (layer "B.Cu") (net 22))
 (segment (start 37.176524 49.754976) (end 37.891238 49.040262) (width 0.255524) (layer "B.Cu") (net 22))
 (segment (start 35.470462 49.754976) (end 37.176524 49.754976) (width 0.255524) (layer "B.Cu") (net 22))
 (segment (start 38.941262 35.808738) (end 38.941262 36.299224) (width 0.255524) (layer "B.Cu") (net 22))
 (segment (start 39.75 35) (end 38.941262 35.808738) (width 0.255524) (layer "B.Cu") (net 22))
 (segment (start 37.891238 49.040262) (end 37.891238 48.484738) (width 0.255524) (layer "B.Cu") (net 22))
 (segment (start 33.523762 38.216724) (end 33.523762 47.808276) (width 0.255524) (layer "B.Cu") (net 22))
 (segment (start 37.911724 37.328762) (end 34.411724 37.328762) (width 0.255524) (layer "B.Cu") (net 22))
 (segment (start 38.941262 36.299224) (end 37.911724 37.328762) (width 0.255524) (layer "B.Cu") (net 22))
 (segment (start 33.523762 47.808276) (end 35.470462 49.754976) (width 0.255524) (layer "B.Cu") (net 22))
 (segment (start 34.411724 37.328762) (end 33.523762 38.216724) (width 0.255524) (layer "B.Cu") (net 22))
 (segment (start 42.067862 43.517862) (end 41.948224 43.6375) (width 0.255524) (layer "F.Cu") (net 24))
 (segment (start 39.773762 49.466724) (end 39.773762 43.966724) (width 0.255524) (layer "F.Cu") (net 24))
 (segment (start 39.1725 50.732499) (end 39.113762 50.673761) (width 0.255524) (layer "F.Cu") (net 24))
 (segment (start 41.2875 42.6375) (end 41.948224 42.6375) (width 0.255524) (layer "F.Cu") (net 24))
 (segment (start 41.948224 42.6375) (end 42.067862 42.757138) (width 0.255524) (layer "F.Cu") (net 24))
 (segment (start 39.773762 43.966724) (end 40.161724 43.578762) (width 0.255524) (layer "F.Cu") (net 24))
 (segment (start 40.161724 43.578762) (end 40.403761 43.578762) (width 0.255524) (layer "F.Cu") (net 24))
 (segment (start 41.948224 43.6375) (end 41.2875 43.6375) (width 0.255524) (layer "F.Cu") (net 24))
 (segment (start 42.067862 42.757138) (end 42.067862 43.517862) (width 0.255524) (layer "F.Cu") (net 24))
 (segment (start 40.403761 43.578762) (end 40.462499 43.6375) (width 0.255524) (layer "F.Cu") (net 24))
 (segment (start 39.113762 50.673761) (end 39.113762 50.126724) (width 0.255524) (layer "F.Cu") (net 24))
 (segment (start 39.113762 50.126724) (end 39.773762 49.466724) (width 0.255524) (layer "F.Cu") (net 24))
 (segment (start 40.462499 43.6375) (end 41.2875 43.6375) (width 0.255524) (layer "F.Cu") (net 24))
 (segment (start 39.1725 51.2275) (end 39.1725 50.732499) (width 0.255524) (layer "F.Cu") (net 24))
 (segment (start 42.067862 63.017862) (end 42.067862 62.257138) (width 0.255524) (layer "F.Cu") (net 12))
 (segment (start 39.907533 62.196238) (end 40.403761 62.196238) (width 0.255524) (layer "F.Cu") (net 12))
 (segment (start 40.386239 51.946238) (end 41.661724 51.946238) (width 0.255524) (layer "F.Cu") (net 12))
 (segment (start 42.067862 62.257138) (end 41.948224 62.1375) (width 0.255524) (layer "F.Cu") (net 12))
 (segment (start 40.403761 62.196238) (end 40.462499 62.1375) (width 0.255524) (layer "F.Cu") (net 12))
 (segment (start 42.773762 55.716724) (end 39.465024 59.025462) (width 0.255524) (layer "F.Cu") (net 12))
 (segment (start 39.465024 61.753729) (end 39.907533 62.196238) (width 0.255524) (layer "F.Cu") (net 12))
 (segment (start 41.948224 62.1375) (end 41.2875 62.1375) (width 0.255524) (layer "F.Cu") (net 12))
 (segment (start 39.8325 51.8875) (end 40.327501 51.8875) (width 0.255524) (layer "F.Cu") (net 12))
 (segment (start 40.462499 62.1375) (end 41.2875 62.1375) (width 0.255524) (layer "F.Cu") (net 12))
 (segment (start 41.948224 63.1375) (end 42.067862 63.017862) (width 0.255524) (layer "F.Cu") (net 12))
 (segment (start 41.661724 51.946238) (end 42.773762 53.058276) (width 0.255524) (layer "F.Cu") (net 12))
 (segment (start 42.773762 53.058276) (end 42.773762 55.716724) (width 0.255524) (layer "F.Cu") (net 12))
 (segment (start 41.2875 63.1375) (end 41.948224 63.1375) (width 0.255524) (layer "F.Cu") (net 12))
 (segment (start 40.327501 51.8875) (end 40.386239 51.946238) (width 0.255524) (layer "F.Cu") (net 12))
 (segment (start 39.465024 59.025462) (end 39.465024 61.753729) (width 0.255524) (layer "F.Cu") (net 12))
 (segment (start 39.1725 54.0475) (end 39.1725 54.542501) (width 0.255524) (layer "F.Cu") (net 31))
 (segment (start 35.432138 42.757138) (end 35.551776 42.6375) (width 0.255524) (layer "F.Cu") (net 31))
 (segment (start 37.891238 46.828762) (end 37.891238 43.966724) (width 0.255524) (layer "F.Cu") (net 31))
 (segment (start 35.432138 43.517862) (end 35.432138 42.757138) (width 0.255524) (layer "F.Cu") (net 31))
 (segment (start 37.891238 43.966724) (end 37.503276 43.578762) (width 0.255524) (layer "F.Cu") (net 31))
 (segment (start 39.113762 55.335752) (end 38.42949 56.020024) (width 0.255524) (layer "F.Cu") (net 31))
 (segment (start 35.715024 56.020024) (end 34.449976 54.754976) (width 0.255524) (layer "F.Cu") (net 31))
 (segment (start 35.551776 43.6375) (end 35.432138 43.517862) (width 0.255524) (layer "F.Cu") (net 31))
 (segment (start 37.503276 43.578762) (end 37.096239 43.578762) (width 0.255524) (layer "F.Cu") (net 31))
 (segment (start 36.2125 43.6375) (end 35.551776 43.6375) (width 0.255524) (layer "F.Cu") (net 31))
 (segment (start 39.1725 54.542501) (end 39.113762 54.601239) (width 0.255524) (layer "F.Cu") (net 31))
 (segment (start 37.096239 43.578762) (end 37.037501 43.6375) (width 0.255524) (layer "F.Cu") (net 31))
 (segment (start 34.449976 50.270024) (end 37.891238 46.828762) (width 0.255524) (layer "F.Cu") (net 31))
 (segment (start 34.449976 54.754976) (end 34.449976 50.270024) (width 0.255524) (layer "F.Cu") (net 31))
 (segment (start 35.551776 42.6375) (end 36.2125 42.6375) (width 0.255524) (layer "F.Cu") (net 31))
 (segment (start 37.037501 43.6375) (end 36.2125 43.6375) (width 0.255524) (layer "F.Cu") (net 31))
 (segment (start 39.113762 54.601239) (end 39.113762 55.335752) (width 0.255524) (layer "F.Cu") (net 31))
 (segment (start 38.42949 56.020024) (end 35.715024 56.020024) (width 0.255524) (layer "F.Cu") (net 31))
 (segment (start 38.215024 58.525462) (end 38.215024 62.816432) (width 0.255524) (layer "F.Cu") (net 16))
 (segment (start 36.671238 63.578762) (end 36.6125 63.6375) (width 0.255524) (layer "F.Cu") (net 16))
 (segment (start 38.215024 62.816432) (end 37.452694 63.578762) (width 0.255524) (layer "F.Cu") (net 16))
 (segment (start 41.523762 53.558276) (end 41.523762 55.216724) (width 0.255524) (layer "F.Cu") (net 16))
 (segment (start 35.432138 62.757138) (end 35.432138 63.517862) (width 0.255524) (layer "F.Cu") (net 16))
 (segment (start 35.551776 63.6375) (end 36.2125 63.6375) (width 0.255524) (layer "F.Cu") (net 16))
 (segment (start 40.327501 52.8875) (end 40.386239 52.946238) (width 0.255524) (layer "F.Cu") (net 16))
 (segment (start 37.452694 63.578762) (end 36.671238 63.578762) (width 0.255524) (layer "F.Cu") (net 16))
 (segment (start 35.551776 62.6375) (end 35.432138 62.757138) (width 0.255524) (layer "F.Cu") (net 16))
 (segment (start 36.6125 63.6375) (end 36.2125 63.6375) (width 0.255524) (layer "F.Cu") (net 16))
 (segment (start 36.2125 62.6375) (end 35.551776 62.6375) (width 0.255524) (layer "F.Cu") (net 16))
 (segment (start 40.386239 52.946238) (end 40.911724 52.946238) (width 0.255524) (layer "F.Cu") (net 16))
 (segment (start 40.911724 52.946238) (end 41.523762 53.558276) (width 0.255524) (layer "F.Cu") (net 16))
 (segment (start 39.8325 52.8875) (end 40.327501 52.8875) (width 0.255524) (layer "F.Cu") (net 16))
 (segment (start 35.432138 63.517862) (end 35.551776 63.6375) (width 0.255524) (layer "F.Cu") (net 16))
 (segment (start 41.523762 55.216724) (end 38.215024 58.525462) (width 0.255524) (layer "F.Cu") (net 16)))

